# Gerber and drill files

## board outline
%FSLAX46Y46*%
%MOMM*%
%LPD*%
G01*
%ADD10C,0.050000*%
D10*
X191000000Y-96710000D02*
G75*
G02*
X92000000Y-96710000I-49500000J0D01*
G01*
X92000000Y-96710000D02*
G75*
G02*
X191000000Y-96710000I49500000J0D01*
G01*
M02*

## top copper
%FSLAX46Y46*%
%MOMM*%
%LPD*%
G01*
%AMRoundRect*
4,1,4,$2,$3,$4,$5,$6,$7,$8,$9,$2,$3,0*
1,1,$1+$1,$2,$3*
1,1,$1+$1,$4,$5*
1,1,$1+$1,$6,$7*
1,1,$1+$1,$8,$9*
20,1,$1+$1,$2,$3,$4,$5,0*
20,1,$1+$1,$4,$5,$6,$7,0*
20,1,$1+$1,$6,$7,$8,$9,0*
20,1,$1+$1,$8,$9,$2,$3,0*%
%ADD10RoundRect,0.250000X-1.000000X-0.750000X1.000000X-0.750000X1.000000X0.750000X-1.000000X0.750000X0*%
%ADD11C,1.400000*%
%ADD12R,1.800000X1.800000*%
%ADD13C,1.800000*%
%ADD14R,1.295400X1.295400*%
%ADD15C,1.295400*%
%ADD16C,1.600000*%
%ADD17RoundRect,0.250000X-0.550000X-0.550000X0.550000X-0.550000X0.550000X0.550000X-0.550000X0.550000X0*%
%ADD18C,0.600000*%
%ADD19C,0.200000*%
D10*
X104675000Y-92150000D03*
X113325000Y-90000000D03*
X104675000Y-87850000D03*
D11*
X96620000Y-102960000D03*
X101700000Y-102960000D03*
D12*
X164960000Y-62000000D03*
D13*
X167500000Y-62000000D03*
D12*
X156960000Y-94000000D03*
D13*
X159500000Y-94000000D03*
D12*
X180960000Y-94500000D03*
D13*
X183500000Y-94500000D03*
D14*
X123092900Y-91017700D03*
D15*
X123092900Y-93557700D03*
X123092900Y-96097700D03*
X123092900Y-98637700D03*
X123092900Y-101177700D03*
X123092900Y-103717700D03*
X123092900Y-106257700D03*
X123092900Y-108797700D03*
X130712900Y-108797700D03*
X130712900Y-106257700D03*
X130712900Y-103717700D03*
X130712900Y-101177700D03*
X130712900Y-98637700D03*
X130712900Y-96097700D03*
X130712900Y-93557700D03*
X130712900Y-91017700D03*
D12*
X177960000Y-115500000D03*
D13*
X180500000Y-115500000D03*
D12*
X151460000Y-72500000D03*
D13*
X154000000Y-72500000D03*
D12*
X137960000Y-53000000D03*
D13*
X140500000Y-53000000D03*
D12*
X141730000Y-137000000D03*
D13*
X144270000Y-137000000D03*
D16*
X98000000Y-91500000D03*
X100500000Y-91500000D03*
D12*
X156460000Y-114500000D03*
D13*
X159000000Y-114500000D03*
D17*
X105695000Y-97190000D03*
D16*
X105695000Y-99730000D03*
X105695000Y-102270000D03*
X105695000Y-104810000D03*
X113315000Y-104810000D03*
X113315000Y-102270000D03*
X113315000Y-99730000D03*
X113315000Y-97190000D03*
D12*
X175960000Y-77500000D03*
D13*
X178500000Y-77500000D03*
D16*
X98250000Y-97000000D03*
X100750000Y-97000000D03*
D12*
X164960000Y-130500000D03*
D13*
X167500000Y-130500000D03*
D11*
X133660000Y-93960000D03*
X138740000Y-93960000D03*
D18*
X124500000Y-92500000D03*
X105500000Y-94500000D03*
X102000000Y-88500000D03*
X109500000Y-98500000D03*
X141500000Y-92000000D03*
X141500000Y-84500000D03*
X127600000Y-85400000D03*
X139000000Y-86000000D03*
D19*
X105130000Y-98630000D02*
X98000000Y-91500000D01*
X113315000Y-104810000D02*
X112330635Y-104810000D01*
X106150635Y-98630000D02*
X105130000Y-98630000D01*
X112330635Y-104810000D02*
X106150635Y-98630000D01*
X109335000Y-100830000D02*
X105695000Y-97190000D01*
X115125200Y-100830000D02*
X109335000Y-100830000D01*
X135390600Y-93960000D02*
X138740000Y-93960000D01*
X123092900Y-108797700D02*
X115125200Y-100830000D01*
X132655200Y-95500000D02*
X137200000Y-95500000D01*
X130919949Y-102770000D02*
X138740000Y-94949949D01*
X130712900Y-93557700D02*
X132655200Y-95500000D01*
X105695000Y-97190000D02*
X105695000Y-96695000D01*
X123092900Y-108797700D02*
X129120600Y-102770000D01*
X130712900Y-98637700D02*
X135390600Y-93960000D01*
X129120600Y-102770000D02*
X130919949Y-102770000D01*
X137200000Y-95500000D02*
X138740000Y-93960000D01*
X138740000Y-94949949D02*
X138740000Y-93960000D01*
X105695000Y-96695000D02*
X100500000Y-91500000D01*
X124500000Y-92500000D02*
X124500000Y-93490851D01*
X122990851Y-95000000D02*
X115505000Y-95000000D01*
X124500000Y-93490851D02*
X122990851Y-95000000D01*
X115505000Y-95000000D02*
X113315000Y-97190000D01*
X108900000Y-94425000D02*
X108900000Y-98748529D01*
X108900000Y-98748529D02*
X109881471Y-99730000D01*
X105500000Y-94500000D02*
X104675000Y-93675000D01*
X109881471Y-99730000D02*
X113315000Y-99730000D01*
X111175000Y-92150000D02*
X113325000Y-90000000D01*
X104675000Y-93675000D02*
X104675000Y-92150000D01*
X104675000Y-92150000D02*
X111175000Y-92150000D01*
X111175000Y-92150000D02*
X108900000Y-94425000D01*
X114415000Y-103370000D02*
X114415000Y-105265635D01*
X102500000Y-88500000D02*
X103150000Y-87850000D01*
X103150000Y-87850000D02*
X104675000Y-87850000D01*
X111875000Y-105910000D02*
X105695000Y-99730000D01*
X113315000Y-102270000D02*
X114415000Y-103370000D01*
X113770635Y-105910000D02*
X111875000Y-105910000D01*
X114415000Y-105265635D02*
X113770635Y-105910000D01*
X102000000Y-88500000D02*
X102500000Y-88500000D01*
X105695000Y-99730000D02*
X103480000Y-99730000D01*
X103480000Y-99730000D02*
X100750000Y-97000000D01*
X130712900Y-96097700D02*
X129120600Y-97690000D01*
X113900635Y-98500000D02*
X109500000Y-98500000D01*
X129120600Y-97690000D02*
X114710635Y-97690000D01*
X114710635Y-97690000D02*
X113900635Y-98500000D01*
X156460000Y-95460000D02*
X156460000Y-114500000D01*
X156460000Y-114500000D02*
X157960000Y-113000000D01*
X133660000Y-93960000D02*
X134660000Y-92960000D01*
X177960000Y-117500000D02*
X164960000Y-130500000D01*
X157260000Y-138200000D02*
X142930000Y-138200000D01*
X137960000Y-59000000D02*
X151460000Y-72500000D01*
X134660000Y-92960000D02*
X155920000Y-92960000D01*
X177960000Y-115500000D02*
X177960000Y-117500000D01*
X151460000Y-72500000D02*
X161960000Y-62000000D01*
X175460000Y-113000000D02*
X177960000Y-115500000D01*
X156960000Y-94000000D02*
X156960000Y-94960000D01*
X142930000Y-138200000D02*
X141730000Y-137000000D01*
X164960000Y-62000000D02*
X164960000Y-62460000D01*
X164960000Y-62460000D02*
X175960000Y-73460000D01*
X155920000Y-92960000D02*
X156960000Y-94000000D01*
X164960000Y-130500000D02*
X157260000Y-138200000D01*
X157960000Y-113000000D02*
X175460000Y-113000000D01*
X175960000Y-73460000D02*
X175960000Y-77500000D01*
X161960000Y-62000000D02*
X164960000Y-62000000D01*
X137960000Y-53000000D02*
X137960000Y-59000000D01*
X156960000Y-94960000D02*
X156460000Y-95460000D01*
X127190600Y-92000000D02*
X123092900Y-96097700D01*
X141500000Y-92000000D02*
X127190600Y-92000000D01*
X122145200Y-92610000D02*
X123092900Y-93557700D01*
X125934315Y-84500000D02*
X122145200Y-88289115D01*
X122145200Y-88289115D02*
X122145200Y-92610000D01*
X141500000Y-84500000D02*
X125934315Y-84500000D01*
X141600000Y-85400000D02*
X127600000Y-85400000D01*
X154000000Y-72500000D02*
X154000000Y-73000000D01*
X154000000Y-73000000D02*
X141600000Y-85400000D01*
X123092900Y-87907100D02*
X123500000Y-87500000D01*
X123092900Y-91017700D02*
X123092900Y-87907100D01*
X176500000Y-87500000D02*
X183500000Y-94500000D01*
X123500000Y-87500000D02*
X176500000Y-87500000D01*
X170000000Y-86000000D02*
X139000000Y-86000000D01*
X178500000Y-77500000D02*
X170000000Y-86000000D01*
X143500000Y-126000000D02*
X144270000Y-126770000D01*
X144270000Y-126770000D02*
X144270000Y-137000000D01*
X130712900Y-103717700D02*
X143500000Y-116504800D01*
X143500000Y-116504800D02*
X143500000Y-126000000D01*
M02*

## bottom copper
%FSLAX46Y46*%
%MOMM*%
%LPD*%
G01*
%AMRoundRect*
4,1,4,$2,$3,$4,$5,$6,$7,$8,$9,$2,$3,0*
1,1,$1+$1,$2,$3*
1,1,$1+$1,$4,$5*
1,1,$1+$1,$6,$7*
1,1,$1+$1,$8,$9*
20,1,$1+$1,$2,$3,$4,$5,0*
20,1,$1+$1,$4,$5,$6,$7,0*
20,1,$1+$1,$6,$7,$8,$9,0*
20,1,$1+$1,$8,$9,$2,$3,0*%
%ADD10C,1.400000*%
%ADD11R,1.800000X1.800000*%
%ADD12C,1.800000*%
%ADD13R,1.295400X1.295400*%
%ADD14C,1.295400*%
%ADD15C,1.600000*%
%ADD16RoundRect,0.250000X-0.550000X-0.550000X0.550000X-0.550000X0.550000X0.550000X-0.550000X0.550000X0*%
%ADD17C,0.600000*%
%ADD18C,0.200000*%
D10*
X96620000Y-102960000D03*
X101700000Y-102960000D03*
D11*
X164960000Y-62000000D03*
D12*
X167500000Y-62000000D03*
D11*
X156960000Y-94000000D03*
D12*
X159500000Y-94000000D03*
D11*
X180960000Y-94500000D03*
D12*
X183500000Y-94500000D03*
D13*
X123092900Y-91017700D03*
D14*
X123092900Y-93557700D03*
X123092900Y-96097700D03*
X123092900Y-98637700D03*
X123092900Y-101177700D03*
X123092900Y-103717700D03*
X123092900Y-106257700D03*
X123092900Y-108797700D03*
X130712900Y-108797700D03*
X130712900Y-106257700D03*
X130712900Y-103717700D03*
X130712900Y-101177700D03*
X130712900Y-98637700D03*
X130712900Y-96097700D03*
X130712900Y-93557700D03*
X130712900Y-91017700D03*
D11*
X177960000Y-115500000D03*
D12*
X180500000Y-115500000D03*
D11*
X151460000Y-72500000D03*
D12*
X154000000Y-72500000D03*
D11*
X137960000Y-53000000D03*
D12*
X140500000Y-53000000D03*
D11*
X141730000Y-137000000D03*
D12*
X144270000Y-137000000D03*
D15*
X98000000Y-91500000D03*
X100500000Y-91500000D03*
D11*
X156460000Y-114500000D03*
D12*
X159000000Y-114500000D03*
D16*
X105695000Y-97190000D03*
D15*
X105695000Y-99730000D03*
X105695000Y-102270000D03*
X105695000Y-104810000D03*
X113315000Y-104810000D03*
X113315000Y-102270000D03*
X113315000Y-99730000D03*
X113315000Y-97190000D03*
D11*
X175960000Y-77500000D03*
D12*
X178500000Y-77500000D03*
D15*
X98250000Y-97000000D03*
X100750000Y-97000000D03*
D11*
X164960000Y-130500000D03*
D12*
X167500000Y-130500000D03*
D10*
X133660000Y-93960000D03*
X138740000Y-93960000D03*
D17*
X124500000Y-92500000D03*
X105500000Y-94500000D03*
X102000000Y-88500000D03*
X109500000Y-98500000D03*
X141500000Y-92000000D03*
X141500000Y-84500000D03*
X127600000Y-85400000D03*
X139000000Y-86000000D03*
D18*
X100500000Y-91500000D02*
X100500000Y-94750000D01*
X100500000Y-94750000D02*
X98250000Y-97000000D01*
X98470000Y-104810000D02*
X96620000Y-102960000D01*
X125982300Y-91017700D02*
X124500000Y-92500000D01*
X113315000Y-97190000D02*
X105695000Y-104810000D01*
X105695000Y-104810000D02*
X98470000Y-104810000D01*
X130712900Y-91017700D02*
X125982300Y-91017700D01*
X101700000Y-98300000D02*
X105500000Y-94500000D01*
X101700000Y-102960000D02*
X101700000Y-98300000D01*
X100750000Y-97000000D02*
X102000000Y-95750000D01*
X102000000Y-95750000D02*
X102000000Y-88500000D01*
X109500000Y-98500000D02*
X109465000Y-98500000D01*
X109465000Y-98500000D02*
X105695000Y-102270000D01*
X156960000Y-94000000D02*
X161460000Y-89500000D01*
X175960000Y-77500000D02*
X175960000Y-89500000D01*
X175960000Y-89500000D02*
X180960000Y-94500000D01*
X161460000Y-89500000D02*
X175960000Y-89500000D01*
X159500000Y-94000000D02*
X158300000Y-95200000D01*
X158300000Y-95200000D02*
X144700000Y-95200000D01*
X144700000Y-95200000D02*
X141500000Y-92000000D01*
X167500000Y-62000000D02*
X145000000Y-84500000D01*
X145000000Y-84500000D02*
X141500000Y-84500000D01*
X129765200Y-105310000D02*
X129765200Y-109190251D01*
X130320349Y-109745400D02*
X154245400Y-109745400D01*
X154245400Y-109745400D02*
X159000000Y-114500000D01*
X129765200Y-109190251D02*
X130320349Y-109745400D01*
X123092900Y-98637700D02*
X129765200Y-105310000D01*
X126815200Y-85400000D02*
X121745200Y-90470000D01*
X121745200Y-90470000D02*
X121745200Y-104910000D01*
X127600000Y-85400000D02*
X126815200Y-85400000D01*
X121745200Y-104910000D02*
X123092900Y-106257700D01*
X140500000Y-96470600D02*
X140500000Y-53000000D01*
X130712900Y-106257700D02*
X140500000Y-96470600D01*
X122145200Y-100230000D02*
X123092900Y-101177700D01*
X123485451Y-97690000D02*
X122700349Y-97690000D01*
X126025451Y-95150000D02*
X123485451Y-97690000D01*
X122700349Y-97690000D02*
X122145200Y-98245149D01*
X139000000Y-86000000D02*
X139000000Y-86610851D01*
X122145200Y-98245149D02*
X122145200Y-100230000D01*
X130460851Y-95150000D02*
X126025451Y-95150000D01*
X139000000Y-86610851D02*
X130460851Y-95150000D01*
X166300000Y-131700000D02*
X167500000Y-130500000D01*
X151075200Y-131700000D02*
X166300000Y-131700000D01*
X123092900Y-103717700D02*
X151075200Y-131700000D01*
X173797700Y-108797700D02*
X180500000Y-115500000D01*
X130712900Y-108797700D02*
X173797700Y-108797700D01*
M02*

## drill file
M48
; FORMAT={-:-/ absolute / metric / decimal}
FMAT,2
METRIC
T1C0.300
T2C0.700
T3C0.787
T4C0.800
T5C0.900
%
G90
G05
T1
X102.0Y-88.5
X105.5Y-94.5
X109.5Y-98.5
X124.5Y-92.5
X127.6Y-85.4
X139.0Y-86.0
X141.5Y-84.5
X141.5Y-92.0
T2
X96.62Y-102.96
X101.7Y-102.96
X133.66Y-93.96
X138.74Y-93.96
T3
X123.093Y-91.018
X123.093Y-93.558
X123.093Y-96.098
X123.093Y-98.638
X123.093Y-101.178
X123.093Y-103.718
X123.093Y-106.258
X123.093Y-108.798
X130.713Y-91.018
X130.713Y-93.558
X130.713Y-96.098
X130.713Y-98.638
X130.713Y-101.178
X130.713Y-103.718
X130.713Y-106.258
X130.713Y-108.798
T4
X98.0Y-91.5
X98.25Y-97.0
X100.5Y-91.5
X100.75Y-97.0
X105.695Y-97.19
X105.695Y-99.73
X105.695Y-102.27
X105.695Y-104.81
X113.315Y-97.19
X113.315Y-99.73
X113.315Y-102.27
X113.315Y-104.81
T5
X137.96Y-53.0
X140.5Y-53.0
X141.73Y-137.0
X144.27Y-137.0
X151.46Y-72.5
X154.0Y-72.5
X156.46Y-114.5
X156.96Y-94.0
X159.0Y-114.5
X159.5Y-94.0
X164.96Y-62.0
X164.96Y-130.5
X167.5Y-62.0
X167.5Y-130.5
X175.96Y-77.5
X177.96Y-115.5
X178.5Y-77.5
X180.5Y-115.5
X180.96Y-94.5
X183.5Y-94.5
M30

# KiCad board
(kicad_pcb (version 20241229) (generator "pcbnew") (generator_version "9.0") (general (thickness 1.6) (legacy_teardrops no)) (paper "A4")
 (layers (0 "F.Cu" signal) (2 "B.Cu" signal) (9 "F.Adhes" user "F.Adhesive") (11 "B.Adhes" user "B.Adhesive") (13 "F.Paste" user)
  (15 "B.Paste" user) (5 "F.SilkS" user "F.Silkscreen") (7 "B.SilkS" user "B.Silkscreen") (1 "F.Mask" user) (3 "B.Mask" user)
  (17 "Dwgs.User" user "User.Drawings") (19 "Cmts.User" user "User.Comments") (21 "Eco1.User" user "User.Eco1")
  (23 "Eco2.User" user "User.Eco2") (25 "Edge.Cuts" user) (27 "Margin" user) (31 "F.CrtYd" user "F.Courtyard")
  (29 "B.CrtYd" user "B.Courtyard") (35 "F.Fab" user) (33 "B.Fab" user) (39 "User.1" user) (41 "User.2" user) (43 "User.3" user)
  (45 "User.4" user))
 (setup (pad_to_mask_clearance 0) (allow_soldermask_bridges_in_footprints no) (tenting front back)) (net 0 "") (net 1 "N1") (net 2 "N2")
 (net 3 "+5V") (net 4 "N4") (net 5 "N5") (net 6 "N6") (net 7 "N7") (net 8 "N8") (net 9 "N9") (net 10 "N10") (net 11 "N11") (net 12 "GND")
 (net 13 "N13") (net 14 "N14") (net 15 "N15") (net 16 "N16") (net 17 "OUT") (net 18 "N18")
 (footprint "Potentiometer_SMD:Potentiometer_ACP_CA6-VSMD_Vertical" (layer "F.Cu") (at 109 90)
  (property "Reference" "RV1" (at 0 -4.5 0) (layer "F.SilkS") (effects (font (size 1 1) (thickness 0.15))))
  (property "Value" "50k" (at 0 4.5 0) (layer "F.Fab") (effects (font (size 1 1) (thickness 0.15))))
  (pad "1" smd roundrect (at -4.325 2.15) (size 2.5 2) (layers "F.Cu" "F.Mask" "F.Paste") (roundrect_rratio 0.125) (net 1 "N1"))
  (pad "2" smd roundrect (at 4.325 0) (size 2.5 2) (layers "F.Cu" "F.Mask" "F.Paste") (roundrect_rratio 0.125) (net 1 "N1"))
  (pad "3" smd roundrect (at -4.325 -2.15) (size 2.5 2) (layers "F.Cu" "F.Mask" "F.Paste") (roundrect_rratio 0.125) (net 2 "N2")))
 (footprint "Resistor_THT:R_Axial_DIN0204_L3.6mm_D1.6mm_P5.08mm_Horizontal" (layer "F.Cu") (at 96.62 102.96)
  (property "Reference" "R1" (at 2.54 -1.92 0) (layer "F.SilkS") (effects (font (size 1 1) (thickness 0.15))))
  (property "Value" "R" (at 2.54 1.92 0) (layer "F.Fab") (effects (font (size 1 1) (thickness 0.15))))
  (pad "1" thru_hole circle (at 0 0) (size 1.4 1.4) (drill 0.7) (layers "*.Cu" "*.Mask") (remove_unused_layers no) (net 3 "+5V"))
  (pad "2" thru_hole circle (at 5.08 0) (size 1.4 1.4) (drill 0.7) (layers "*.Cu" "*.Mask") (remove_unused_layers no) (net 1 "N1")))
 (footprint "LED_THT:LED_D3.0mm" (layer "F.Cu") (at 164.96 62)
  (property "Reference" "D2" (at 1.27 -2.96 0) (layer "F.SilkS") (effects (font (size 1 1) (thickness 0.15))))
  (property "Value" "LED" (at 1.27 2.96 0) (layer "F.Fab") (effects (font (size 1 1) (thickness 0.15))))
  (pad "1" thru_hole rect (at 0 0) (size 1.8 1.8) (drill 0.9) (layers "*.Cu" "*.Mask") (remove_unused_layers no) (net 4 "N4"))
  (pad "2" thru_hole circle (at 2.54 0) (size 1.8 1.8) (drill 0.9) (layers "*.Cu" "*.Mask") (remove_unused_layers no) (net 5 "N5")))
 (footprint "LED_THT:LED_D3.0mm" (layer "F.Cu") (at 156.96 94)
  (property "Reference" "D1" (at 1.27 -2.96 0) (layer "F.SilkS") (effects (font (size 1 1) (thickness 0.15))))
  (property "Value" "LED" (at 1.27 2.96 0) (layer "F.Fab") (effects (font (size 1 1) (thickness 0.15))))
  (pad "1" thru_hole rect (at 0 0) (size 1.8 1.8) (drill 0.9) (layers "*.Cu" "*.Mask") (remove_unused_layers no) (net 4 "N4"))
  (pad "2" thru_hole circle (at 2.54 0) (size 1.8 1.8) (drill 0.9) (layers "*.Cu" "*.Mask") (remove_unused_layers no) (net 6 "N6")))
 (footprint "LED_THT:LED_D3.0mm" (layer "F.Cu") (at 180.96 94.5)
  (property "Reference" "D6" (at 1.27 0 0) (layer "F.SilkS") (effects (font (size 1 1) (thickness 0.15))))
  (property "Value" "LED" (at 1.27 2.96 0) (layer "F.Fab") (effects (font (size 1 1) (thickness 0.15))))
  (pad "1" thru_hole rect (at 0 0) (size 1.8 1.8) (drill 0.9) (layers "*.Cu" "*.Mask") (remove_unused_layers no) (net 4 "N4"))
  (pad "2" thru_hole circle (at 2.54 0) (size 1.8 1.8) (drill 0.9) (layers "*.Cu" "*.Mask") (remove_unused_layers no) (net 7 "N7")))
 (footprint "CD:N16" (layer "F.Cu") (at 123.0929 91.0177)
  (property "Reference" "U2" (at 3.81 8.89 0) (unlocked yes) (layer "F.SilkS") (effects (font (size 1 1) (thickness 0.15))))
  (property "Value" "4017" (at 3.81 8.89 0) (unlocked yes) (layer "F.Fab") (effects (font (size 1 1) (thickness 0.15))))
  (pad "1" thru_hole rect (at 0 0) (size 1.2954 1.2954) (drill 0.7874) (layers "*.Cu" "*.Mask") (remove_unused_layers no) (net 7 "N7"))
  (pad "2" thru_hole circle (at 0 2.54) (size 1.2954 1.2954) (drill 0.7874) (layers "*.Cu" "*.Mask") (remove_unused_layers no) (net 5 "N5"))
  (pad "3" thru_hole circle (at 0 5.08) (size 1.2954 1.2954) (drill 0.7874) (layers "*.Cu" "*.Mask") (remove_unused_layers no) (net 6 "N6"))
  (pad "4" thru_hole circle (at 0 7.62) (size 1.2954 1.2954) (drill 0.7874) (layers "*.Cu" "*.Mask") (remove_unused_layers no) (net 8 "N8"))
  (pad "5" thru_hole circle (at 0 10.16) (size 1.2954 1.2954) (drill 0.7874) (layers "*.Cu" "*.Mask") (remove_unused_layers no) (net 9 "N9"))
  (pad "6" thru_hole circle (at 0 12.7) (size 1.2954 1.2954) (drill 0.7874) (layers "*.Cu" "*.Mask") (remove_unused_layers no)
   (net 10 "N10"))
  (pad "7" thru_hole circle (at 0 15.24) (size 1.2954 1.2954) (drill 0.7874) (layers "*.Cu" "*.Mask") (remove_unused_layers no)
   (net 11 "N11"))
  (pad "8" thru_hole circle (at 0 17.78) (size 1.2954 1.2954) (drill 0.7874) (layers "*.Cu" "*.Mask") (remove_unused_layers no)
   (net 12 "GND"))
  (pad "9" thru_hole circle (at 7.62 17.78) (size 1.2954 1.2954) (drill 0.7874) (layers "*.Cu" "*.Mask") (remove_unused_layers no)
   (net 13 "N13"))
  (pad "10" thru_hole circle (at 7.62 15.24) (size 1.2954 1.2954) (drill 0.7874) (layers "*.Cu" "*.Mask") (remove_unused_layers no)
   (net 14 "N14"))
  (pad "11" thru_hole circle (at 7.62 12.7) (size 1.2954 1.2954) (drill 0.7874) (layers "*.Cu" "*.Mask") (remove_unused_layers no)
   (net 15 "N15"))
  (pad "12" thru_hole circle (at 7.62 10.16) (size 1.2954 1.2954) (drill 0.7874) (layers "*.Cu" "*.Mask") (remove_unused_layers no)
   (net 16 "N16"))
  (pad "13" thru_hole circle (at 7.62 7.62) (size 1.2954 1.2954) (drill 0.7874) (layers "*.Cu" "*.Mask") (remove_unused_layers no)
   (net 12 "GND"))
  (pad "14" thru_hole circle (at 7.62 5.08) (size 1.2954 1.2954) (drill 0.7874) (layers "*.Cu" "*.Mask") (remove_unused_layers no)
   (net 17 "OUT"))
  (pad "15" thru_hole circle (at 7.62 2.54) (size 1.2954 1.2954) (drill 0.7874) (layers "*.Cu" "*.Mask") (remove_unused_layers no)
   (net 12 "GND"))
  (pad "16" thru_hole circle (at 7.62 0) (size 1.2954 1.2954) (drill 0.7874) (layers "*.Cu" "*.Mask") (remove_unused_layers no)
   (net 3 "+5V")))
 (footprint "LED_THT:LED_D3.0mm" (layer "F.Cu") (at 177.96 115.5)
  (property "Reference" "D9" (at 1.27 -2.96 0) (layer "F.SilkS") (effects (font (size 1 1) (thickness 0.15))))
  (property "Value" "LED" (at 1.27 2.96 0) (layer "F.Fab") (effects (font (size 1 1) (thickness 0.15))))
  (pad "1" thru_hole rect (at 0 0) (size 1.8 1.8) (drill 0.9) (layers "*.Cu" "*.Mask") (remove_unused_layers no) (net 4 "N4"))
  (pad "2" thru_hole circle (at 2.54 0) (size 1.8 1.8) (drill 0.9) (layers "*.Cu" "*.Mask") (remove_unused_layers no) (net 13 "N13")))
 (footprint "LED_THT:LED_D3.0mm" (layer "F.Cu") (at 151.46 72.5)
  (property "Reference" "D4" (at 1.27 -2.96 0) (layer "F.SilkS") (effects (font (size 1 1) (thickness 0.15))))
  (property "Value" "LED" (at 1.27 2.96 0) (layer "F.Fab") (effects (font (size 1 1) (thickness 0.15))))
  (pad "1" thru_hole rect (at 0 0) (size 1.8 1.8) (drill 0.9) (layers "*.Cu" "*.Mask") (remove_unused_layers no) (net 4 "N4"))
  (pad "2" thru_hole circle (at 2.54 0) (size 1.8 1.8) (drill 0.9) (layers "*.Cu" "*.Mask") (remove_unused_layers no) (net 11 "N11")))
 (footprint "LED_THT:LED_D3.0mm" (layer "F.Cu") (at 137.96 53)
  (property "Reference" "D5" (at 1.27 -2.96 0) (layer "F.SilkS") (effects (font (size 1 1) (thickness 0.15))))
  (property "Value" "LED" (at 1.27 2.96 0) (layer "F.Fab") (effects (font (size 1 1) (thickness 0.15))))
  (pad "1" thru_hole rect (at 0 0) (size 1.8 1.8) (drill 0.9) (layers "*.Cu" "*.Mask") (remove_unused_layers no) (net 4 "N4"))
  (pad "2" thru_hole circle (at 2.54 0) (size 1.8 1.8) (drill 0.9) (layers "*.Cu" "*.Mask") (remove_unused_layers no) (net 14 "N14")))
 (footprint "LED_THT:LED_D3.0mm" (layer "F.Cu") (at 141.73 137)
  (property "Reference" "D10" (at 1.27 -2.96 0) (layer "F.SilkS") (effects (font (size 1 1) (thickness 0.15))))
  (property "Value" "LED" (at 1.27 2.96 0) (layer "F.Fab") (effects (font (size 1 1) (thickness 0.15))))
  (pad "1" thru_hole rect (at 0 0) (size 1.8 1.8) (drill 0.9) (layers "*.Cu" "*.Mask") (remove_unused_layers no) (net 4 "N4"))
  (pad "2" thru_hole circle (at 2.54 0) (size 1.8 1.8) (drill 0.9) (layers "*.Cu" "*.Mask") (remove_unused_layers no) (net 15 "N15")))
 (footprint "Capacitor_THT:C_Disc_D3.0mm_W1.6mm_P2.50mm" (layer "F.Cu") (at 98 91.5)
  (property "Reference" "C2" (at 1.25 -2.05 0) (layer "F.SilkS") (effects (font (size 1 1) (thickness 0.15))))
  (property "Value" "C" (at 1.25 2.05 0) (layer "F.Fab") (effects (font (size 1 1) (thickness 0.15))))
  (pad "1" thru_hole circle (at 0 0) (size 1.6 1.6) (drill 0.8) (layers "*.Cu" "*.Mask") (remove_unused_layers no) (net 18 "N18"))
  (pad "2" thru_hole circle (at 2.5 0) (size 1.6 1.6) (drill 0.8) (layers "*.Cu" "*.Mask") (remove_unused_layers no) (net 12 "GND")))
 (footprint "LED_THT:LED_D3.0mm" (layer "F.Cu") (at 156.46 114.5)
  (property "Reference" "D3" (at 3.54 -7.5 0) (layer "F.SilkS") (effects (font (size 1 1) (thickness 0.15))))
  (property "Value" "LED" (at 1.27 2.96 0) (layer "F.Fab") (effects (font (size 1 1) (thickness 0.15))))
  (pad "1" thru_hole rect (at 0 0) (size 1.8 1.8) (drill 0.9) (layers "*.Cu" "*.Mask") (remove_unused_layers no) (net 4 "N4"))
  (pad "2" thru_hole circle (at 2.54 0) (size 1.8 1.8) (drill 0.9) (layers "*.Cu" "*.Mask") (remove_unused_layers no) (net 8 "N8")))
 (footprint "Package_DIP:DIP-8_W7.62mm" (layer "F.Cu") (at 105.695 97.19)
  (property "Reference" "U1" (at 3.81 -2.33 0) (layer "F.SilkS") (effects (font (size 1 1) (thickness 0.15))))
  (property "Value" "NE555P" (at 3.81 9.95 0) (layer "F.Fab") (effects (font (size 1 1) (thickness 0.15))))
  (pad "1" thru_hole roundrect (at 0 0) (size 1.6 1.6) (drill 0.8) (layers "*.Cu" "*.Mask") (remove_unused_layers no)
   (roundrect_rratio 0.15625) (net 12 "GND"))
  (pad "2" thru_hole circle (at 0 2.54) (size 1.6 1.6) (drill 0.8) (layers "*.Cu" "*.Mask") (remove_unused_layers no) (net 2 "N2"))
  (pad "3" thru_hole circle (at 0 5.08) (size 1.6 1.6) (drill 0.8) (layers "*.Cu" "*.Mask") (remove_unused_layers no) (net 17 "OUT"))
  (pad "4" thru_hole circle (at 0 7.62) (size 1.6 1.6) (drill 0.8) (layers "*.Cu" "*.Mask") (remove_unused_layers no) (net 3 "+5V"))
  (pad "5" thru_hole circle (at 7.62 7.62) (size 1.6 1.6) (drill 0.8) (layers "*.Cu" "*.Mask") (remove_unused_layers no) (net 18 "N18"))
  (pad "6" thru_hole circle (at 7.62 5.08) (size 1.6 1.6) (drill 0.8) (layers "*.Cu" "*.Mask") (remove_unused_layers no) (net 2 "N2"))
  (pad "7" thru_hole circle (at 7.62 2.54) (size 1.6 1.6) (drill 0.8) (layers "*.Cu" "*.Mask") (remove_unused_layers no) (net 1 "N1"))
  (pad "8" thru_hole circle (at 7.62 0) (size 1.6 1.6) (drill 0.8) (layers "*.Cu" "*.Mask") (remove_unused_layers no) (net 3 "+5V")))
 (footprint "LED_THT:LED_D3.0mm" (layer "F.Cu") (at 175.96 77.5)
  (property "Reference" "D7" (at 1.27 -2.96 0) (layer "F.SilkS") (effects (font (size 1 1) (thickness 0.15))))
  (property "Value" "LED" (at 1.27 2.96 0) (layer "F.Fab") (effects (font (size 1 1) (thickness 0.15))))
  (pad "1" thru_hole rect (at 0 0) (size 1.8 1.8) (drill 0.9) (layers "*.Cu" "*.Mask") (remove_unused_layers no) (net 4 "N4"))
  (pad "2" thru_hole circle (at 2.54 0) (size 1.8 1.8) (drill 0.9) (layers "*.Cu" "*.Mask") (remove_unused_layers no) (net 9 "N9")))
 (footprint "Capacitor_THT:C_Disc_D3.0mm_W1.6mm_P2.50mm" (layer "F.Cu") (at 98.25 97)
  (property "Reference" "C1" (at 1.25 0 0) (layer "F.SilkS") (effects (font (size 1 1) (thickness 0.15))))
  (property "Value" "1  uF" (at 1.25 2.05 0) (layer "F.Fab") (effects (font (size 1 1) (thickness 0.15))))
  (pad "1" thru_hole circle (at 0 0) (size 1.6 1.6) (drill 0.8) (layers "*.Cu" "*.Mask") (remove_unused_layers no) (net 12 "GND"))
  (pad "2" thru_hole circle (at 2.5 0) (size 1.6 1.6) (drill 0.8) (layers "*.Cu" "*.Mask") (remove_unused_layers no) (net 2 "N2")))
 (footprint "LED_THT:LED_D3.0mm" (layer "F.Cu") (at 164.96 130.5)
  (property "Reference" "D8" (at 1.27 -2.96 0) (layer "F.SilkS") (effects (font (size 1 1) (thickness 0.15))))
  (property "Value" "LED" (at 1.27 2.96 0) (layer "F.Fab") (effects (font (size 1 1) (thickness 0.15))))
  (pad "1" thru_hole rect (at 0 0) (size 1.8 1.8) (drill 0.9) (layers "*.Cu" "*.Mask") (remove_unused_layers no) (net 4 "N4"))
  (pad "2" thru_hole circle (at 2.54 0) (size 1.8 1.8) (drill 0.9) (layers "*.Cu" "*.Mask") (remove_unused_layers no) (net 10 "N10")))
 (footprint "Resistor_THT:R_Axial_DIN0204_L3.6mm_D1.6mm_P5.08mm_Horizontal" (layer "F.Cu") (at 133.66 93.96)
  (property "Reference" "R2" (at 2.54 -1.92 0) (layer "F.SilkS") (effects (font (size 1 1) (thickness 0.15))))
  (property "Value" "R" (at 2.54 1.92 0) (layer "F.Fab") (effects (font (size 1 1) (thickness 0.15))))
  (pad "1" thru_hole circle (at 0 0) (size 1.4 1.4) (drill 0.7) (layers "*.Cu" "*.Mask") (remove_unused_layers no) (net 4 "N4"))
  (pad "2" thru_hole circle (at 5.08 0) (size 1.4 1.4) (drill 0.7) (layers "*.Cu" "*.Mask") (remove_unused_layers no) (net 12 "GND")))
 (gr_circle (center 141.5 96.71) (end 191 96.71) (stroke (width 0.05) (type default)) (fill no) (layer "Edge.Cuts"))
 (segment (start 105.13 98.63) (end 98 91.5) (width 0.2) (layer "F.Cu") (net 18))
 (segment (start 113.315 104.81) (end 112.330635 104.81) (width 0.2) (layer "F.Cu") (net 18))
 (segment (start 106.150635 98.63) (end 105.13 98.63) (width 0.2) (layer "F.Cu") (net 18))
 (segment (start 112.330635 104.81) (end 106.150635 98.63) (width 0.2) (layer "F.Cu") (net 18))
 (segment (start 109.335 100.83) (end 105.695 97.19) (width 0.2) (layer "F.Cu") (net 12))
 (segment (start 115.1252 100.83) (end 109.335 100.83) (width 0.2) (layer "F.Cu") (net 12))
 (segment (start 135.3906 93.96) (end 138.74 93.96) (width 0.2) (layer "F.Cu") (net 12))
 (segment (start 123.0929 108.7977) (end 115.1252 100.83) (width 0.2) (layer "F.Cu") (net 12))
 (segment (start 132.6552 95.5) (end 137.2 95.5) (width 0.2) (layer "F.Cu") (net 12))
 (segment (start 130.919949 102.77) (end 138.74 94.949949) (width 0.2) (layer "F.Cu") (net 12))
 (segment (start 130.7129 93.5577) (end 132.6552 95.5) (width 0.2) (layer "F.Cu") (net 12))
 (segment (start 105.695 97.19) (end 105.695 96.695) (width 0.2) (layer "F.Cu") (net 12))
 (segment (start 123.0929 108.7977) (end 129.1206 102.77) (width 0.2) (layer "F.Cu") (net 12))
 (segment (start 130.7129 98.6377) (end 135.3906 93.96) (width 0.2) (layer "F.Cu") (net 12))
 (segment (start 129.1206 102.77) (end 130.919949 102.77) (width 0.2) (layer "F.Cu") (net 12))
 (segment (start 137.2 95.5) (end 138.74 93.96) (width 0.2) (layer "F.Cu") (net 12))
 (segment (start 138.74 94.949949) (end 138.74 93.96) (width 0.2) (layer "F.Cu") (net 12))
 (segment (start 105.695 96.695) (end 100.5 91.5) (width 0.2) (layer "F.Cu") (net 12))
 (segment (start 100.5 91.5) (end 100.5 94.75) (width 0.2) (layer "B.Cu") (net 12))
 (segment (start 100.5 94.75) (end 98.25 97) (width 0.2) (layer "B.Cu") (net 12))
 (segment (start 124.5 92.5) (end 124.5 93.490851) (width 0.2) (layer "F.Cu") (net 3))
 (segment (start 122.990851 95) (end 115.505 95) (width 0.2) (layer "F.Cu") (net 3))
 (segment (start 124.5 93.490851) (end 122.990851 95) (width 0.2) (layer "F.Cu") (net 3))
 (segment (start 115.505 95) (end 113.315 97.19) (width 0.2) (layer "F.Cu") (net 3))
 (via (at 124.5 92.5) (size 0.6) (drill 0.3) (layers "F.Cu" "B.Cu") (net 3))
 (segment (start 98.47 104.81) (end 96.62 102.96) (width 0.2) (layer "B.Cu") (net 3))
 (segment (start 125.9823 91.0177) (end 124.5 92.5) (width 0.2) (layer "B.Cu") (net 3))
 (segment (start 113.315 97.19) (end 105.695 104.81) (width 0.2) (layer "B.Cu") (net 3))
 (segment (start 105.695 104.81) (end 98.47 104.81) (width 0.2) (layer "B.Cu") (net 3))
 (segment (start 130.7129 91.0177) (end 125.9823 91.0177) (width 0.2) (layer "B.Cu") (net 3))
 (segment (start 108.9 94.425) (end 108.9 98.748529) (width 0.2) (layer "F.Cu") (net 1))
 (segment (start 108.9 98.748529) (end 109.881471 99.73) (width 0.2) (layer "F.Cu") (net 1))
 (segment (start 105.5 94.5) (end 104.675 93.675) (width 0.2) (layer "F.Cu") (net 1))
 (segment (start 109.881471 99.73) (end 113.315 99.73) (width 0.2) (layer "F.Cu") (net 1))
 (segment (start 111.175 92.15) (end 113.325 90) (width 0.2) (layer "F.Cu") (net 1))
 (segment (start 104.675 93.675) (end 104.675 92.15) (width 0.2) (layer "F.Cu") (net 1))
 (segment (start 104.675 92.15) (end 111.175 92.15) (width 0.2) (layer "F.Cu") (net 1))
 (segment (start 111.175 92.15) (end 108.9 94.425) (width 0.2) (layer "F.Cu") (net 1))
 (via (at 105.5 94.5) (size 0.6) (drill 0.3) (layers "F.Cu" "B.Cu") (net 1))
 (segment (start 101.7 98.3) (end 105.5 94.5) (width 0.2) (layer "B.Cu") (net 1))
 (segment (start 101.7 102.96) (end 101.7 98.3) (width 0.2) (layer "B.Cu") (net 1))
 (segment (start 114.415 103.37) (end 114.415 105.265635) (width 0.2) (layer "F.Cu") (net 2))
 (segment (start 102.5 88.5) (end 103.15 87.85) (width 0.2) (layer "F.Cu") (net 2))
 (segment (start 103.15 87.85) (end 104.675 87.85) (width 0.2) (layer "F.Cu") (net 2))
 (segment (start 111.875 105.91) (end 105.695 99.73) (width 0.2) (layer "F.Cu") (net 2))
 (segment (start 113.315 102.27) (end 114.415 103.37) (width 0.2) (layer "F.Cu") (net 2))
 (segment (start 113.770635 105.91) (end 111.875 105.91) (width 0.2) (layer "F.Cu") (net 2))
 (segment (start 114.415 105.265635) (end 113.770635 105.91) (width 0.2) (layer "F.Cu") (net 2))
 (segment (start 102 88.5) (end 102.5 88.5) (width 0.2) (layer "F.Cu") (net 2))
 (segment (start 105.695 99.73) (end 103.48 99.73) (width 0.2) (layer "F.Cu") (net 2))
 (segment (start 103.48 99.73) (end 100.75 97) (width 0.2) (layer "F.Cu") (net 2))
 (via (at 102 88.5) (size 0.6) (drill 0.3) (layers "F.Cu" "B.Cu") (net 2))
 (segment (start 100.75 97) (end 102 95.75) (width 0.2) (layer "B.Cu") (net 2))
 (segment (start 102 95.75) (end 102 88.5) (width 0.2) (layer "B.Cu") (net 2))
 (segment (start 130.7129 96.0977) (end 129.1206 97.69) (width 0.2) (layer "F.Cu") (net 17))
 (segment (start 113.900635 98.5) (end 109.5 98.5) (width 0.2) (layer "F.Cu") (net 17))
 (segment (start 129.1206 97.69) (end 114.710635 97.69) (width 0.2) (layer "F.Cu") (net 17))
 (segment (start 114.710635 97.69) (end 113.900635 98.5) (width 0.2) (layer "F.Cu") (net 17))
 (via (at 109.5 98.5) (size 0.6) (drill 0.3) (layers "F.Cu" "B.Cu") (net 17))
 (segment (start 109.5 98.5) (end 109.465 98.5) (width 0.2) (layer "B.Cu") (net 17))
 (segment (start 109.465 98.5) (end 105.695 102.27) (width 0.2) (layer "B.Cu") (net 17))
 (segment (start 156.46 95.46) (end 156.46 114.5) (width 0.2) (layer "F.Cu") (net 4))
 (segment (start 156.46 114.5) (end 157.96 113) (width 0.2) (layer "F.Cu") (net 4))
 (segment (start 133.66 93.96) (end 134.66 92.96) (width 0.2) (layer "F.Cu") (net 4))
 (segment (start 177.96 117.5) (end 164.96 130.5) (width 0.2) (layer "F.Cu") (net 4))
 (segment (start 157.26 138.2) (end 142.93 138.2) (width 0.2) (layer "F.Cu") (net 4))
 (segment (start 137.96 59) (end 151.46 72.5) (width 0.2) (layer "F.Cu") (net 4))
 (segment (start 134.66 92.96) (end 155.92 92.96) (width 0.2) (layer "F.Cu") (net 4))
 (segment (start 177.96 115.5) (end 177.96 117.5) (width 0.2) (layer "F.Cu") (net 4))
 (segment (start 151.46 72.5) (end 161.96 62) (width 0.2) (layer "F.Cu") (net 4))
 (segment (start 175.46 113) (end 177.96 115.5) (width 0.2) (layer "F.Cu") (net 4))
 (segment (start 156.96 94) (end 156.96 94.96) (width 0.2) (layer "F.Cu") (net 4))
 (segment (start 142.93 138.2) (end 141.73 137) (width 0.2) (layer "F.Cu") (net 4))
 (segment (start 164.96 62) (end 164.96 62.46) (width 0.2) (layer "F.Cu") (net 4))
 (segment (start 164.96 62.46) (end 175.96 73.46) (width 0.2) (layer "F.Cu") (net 4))
 (segment (start 155.92 92.96) (end 156.96 94) (width 0.2) (layer "F.Cu") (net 4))
 (segment (start 164.96 130.5) (end 157.26 138.2) (width 0.2) (layer "F.Cu") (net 4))
 (segment (start 157.96 113) (end 175.46 113) (width 0.2) (layer "F.Cu") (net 4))
 (segment (start 175.96 73.46) (end 175.96 77.5) (width 0.2) (layer "F.Cu") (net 4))
 (segment (start 161.96 62) (end 164.96 62) (width 0.2) (layer "F.Cu") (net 4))
 (segment (start 137.96 53) (end 137.96 59) (width 0.2) (layer "F.Cu") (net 4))
 (segment (start 156.96 94.96) (end 156.46 95.46) (width 0.2) (layer "F.Cu") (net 4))
 (segment (start 156.96 94) (end 161.46 89.5) (width 0.2) (layer "B.Cu") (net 4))
 (segment (start 175.96 77.5) (end 175.96 89.5) (width 0.2) (layer "B.Cu") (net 4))
 (segment (start 175.96 89.5) (end 180.96 94.5) (width 0.2) (layer "B.Cu") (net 4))
 (segment (start 161.46 89.5) (end 175.96 89.5) (width 0.2) (layer "B.Cu") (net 4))
 (segment (start 127.1906 92) (end 123.0929 96.0977) (width 0.2) (layer "F.Cu") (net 6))
 (segment (start 141.5 92) (end 127.1906 92) (width 0.2) (layer "F.Cu") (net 6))
 (via (at 141.5 92) (size 0.6) (drill 0.3) (layers "F.Cu" "B.Cu") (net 6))
 (segment (start 159.5 94) (end 158.3 95.2) (width 0.2) (layer "B.Cu") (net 6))
 (segment (start 158.3 95.2) (end 144.7 95.2) (width 0.2) (layer "B.Cu") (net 6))
 (segment (start 144.7 95.2) (end 141.5 92) (width 0.2) (layer "B.Cu") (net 6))
 (segment (start 122.1452 92.61) (end 123.0929 93.5577) (width 0.2) (layer "F.Cu") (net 5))
 (segment (start 125.934315 84.5) (end 122.1452 88.289115) (width 0.2) (layer "F.Cu") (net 5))
 (segment (start 122.1452 88.289115) (end 122.1452 92.61) (width 0.2) (layer "F.Cu") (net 5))
 (segment (start 141.5 84.5) (end 125.934315 84.5) (width 0.2) (layer "F.Cu") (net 5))
 (via (at 141.5 84.5) (size 0.6) (drill 0.3) (layers "F.Cu" "B.Cu") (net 5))
 (segment (start 167.5 62) (end 145 84.5) (width 0.2) (layer "B.Cu") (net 5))
 (segment (start 145 84.5) (end 141.5 84.5) (width 0.2) (layer "B.Cu") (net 5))
 (segment (start 129.7652 105.31) (end 129.7652 109.190251) (width 0.2) (layer "B.Cu") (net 8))
 (segment (start 130.320349 109.7454) (end 154.2454 109.7454) (width 0.2) (layer "B.Cu") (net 8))
 (segment (start 154.2454 109.7454) (end 159 114.5) (width 0.2) (layer "B.Cu") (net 8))
 (segment (start 129.7652 109.190251) (end 130.320349 109.7454) (width 0.2) (layer "B.Cu") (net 8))
 (segment (start 123.0929 98.6377) (end 129.7652 105.31) (width 0.2) (layer "B.Cu") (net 8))
 (segment (start 141.6 85.4) (end 127.6 85.4) (width 0.2) (layer "F.Cu") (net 11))
 (segment (start 154 72.5) (end 154 73) (width 0.2) (layer "F.Cu") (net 11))
 (segment (start 154 73) (end 141.6 85.4) (width 0.2) (layer "F.Cu") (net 11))
 (via (at 127.6 85.4) (size 0.6) (drill 0.3) (layers "F.Cu" "B.Cu") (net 11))
 (segment (start 126.8152 85.4) (end 121.7452 90.47) (width 0.2) (layer "B.Cu") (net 11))
 (segment (start 121.7452 90.47) (end 121.7452 104.91) (width 0.2) (layer "B.Cu") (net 11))
 (segment (start 127.6 85.4) (end 126.8152 85.4) (width 0.2) (layer "B.Cu") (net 11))
 (segment (start 121.7452 104.91) (end 123.0929 106.2577) (width 0.2) (layer "B.Cu") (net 11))
 (segment (start 140.5 96.4706) (end 140.5 53) (width 0.2) (layer "B.Cu") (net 14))
 (segment (start 130.7129 106.2577) (end 140.5 96.4706) (width 0.2) (layer "B.Cu") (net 14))
 (segment (start 123.0929 87.9071) (end 123.5 87.5) (width 0.2) (layer "F.Cu") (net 7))
 (segment (start 123.0929 91.0177) (end 123.0929 87.9071) (width 0.2) (layer "F.Cu") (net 7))
 (segment (start 176.5 87.5) (end 183.5 94.5) (width 0.2) (layer "F.Cu") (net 7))
 (segment (start 123.5 87.5) (end 176.5 87.5) (width 0.2) (layer "F.Cu") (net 7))
 (segment (start 170 86) (end 139 86) (width 0.2) (layer "F.Cu") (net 9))
 (segment (start 178.5 77.5) (end 170 86) (width 0.2) (layer "F.Cu") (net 9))
 (via (at 139 86) (size 0.6) (drill 0.3) (layers "F.Cu" "B.Cu") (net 9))
 (segment (start 122.1452 100.23) (end 123.0929 101.1777) (width 0.2) (layer "B.Cu") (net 9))
 (segment (start 123.485451 97.69) (end 122.700349 97.69) (width 0.2) (layer "B.Cu") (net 9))
 (segment (start 126.025451 95.15) (end 123.485451 97.69) (width 0.2) (layer "B.Cu") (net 9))
 (segment (start 122.700349 97.69) (end 122.1452 98.245149) (width 0.2) (layer "B.Cu") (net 9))
 (segment (start 139 86) (end 139 86.610851) (width 0.2) (layer "B.Cu") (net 9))
 (segment (start 122.1452 98.245149) (end 122.1452 100.23) (width 0.2) (layer "B.Cu") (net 9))
 (segment (start 130.460851 95.15) (end 126.025451 95.15) (width 0.2) (layer "B.Cu") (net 9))
 (segment (start 139 86.610851) (end 130.460851 95.15) (width 0.2) (layer "B.Cu") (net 9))
 (segment (start 166.3 131.7) (end 167.5 130.5) (width 0.2) (layer "B.Cu") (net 10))
 (segment (start 151.0752 131.7) (end 166.3 131.7) (width 0.2) (layer "B.Cu") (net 10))
 (segment (start 123.0929 103.7177) (end 151.0752 131.7) (width 0.2) (layer "B.Cu") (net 10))
 (segment (start 173.7977 108.7977) (end 180.5 115.5) (width 0.2) (layer "B.Cu") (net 13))
 (segment (start 130.7129 108.7977) (end 173.7977 108.7977) (width 0.2) (layer "B.Cu") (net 13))
 (segment (start 143.5 126) (end 144.27 126.77) (width 0.2) (layer "F.Cu") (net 15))
 (segment (start 144.27 126.77) (end 144.27 137) (width 0.2) (layer "F.Cu") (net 15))
 (segment (start 130.7129 103.7177) (end 143.5 116.5048) (width 0.2) (layer "F.Cu") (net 15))
 (segment (start 143.5 116.5048) (end 143.5 126) (width 0.2) (layer "F.Cu") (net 15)))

